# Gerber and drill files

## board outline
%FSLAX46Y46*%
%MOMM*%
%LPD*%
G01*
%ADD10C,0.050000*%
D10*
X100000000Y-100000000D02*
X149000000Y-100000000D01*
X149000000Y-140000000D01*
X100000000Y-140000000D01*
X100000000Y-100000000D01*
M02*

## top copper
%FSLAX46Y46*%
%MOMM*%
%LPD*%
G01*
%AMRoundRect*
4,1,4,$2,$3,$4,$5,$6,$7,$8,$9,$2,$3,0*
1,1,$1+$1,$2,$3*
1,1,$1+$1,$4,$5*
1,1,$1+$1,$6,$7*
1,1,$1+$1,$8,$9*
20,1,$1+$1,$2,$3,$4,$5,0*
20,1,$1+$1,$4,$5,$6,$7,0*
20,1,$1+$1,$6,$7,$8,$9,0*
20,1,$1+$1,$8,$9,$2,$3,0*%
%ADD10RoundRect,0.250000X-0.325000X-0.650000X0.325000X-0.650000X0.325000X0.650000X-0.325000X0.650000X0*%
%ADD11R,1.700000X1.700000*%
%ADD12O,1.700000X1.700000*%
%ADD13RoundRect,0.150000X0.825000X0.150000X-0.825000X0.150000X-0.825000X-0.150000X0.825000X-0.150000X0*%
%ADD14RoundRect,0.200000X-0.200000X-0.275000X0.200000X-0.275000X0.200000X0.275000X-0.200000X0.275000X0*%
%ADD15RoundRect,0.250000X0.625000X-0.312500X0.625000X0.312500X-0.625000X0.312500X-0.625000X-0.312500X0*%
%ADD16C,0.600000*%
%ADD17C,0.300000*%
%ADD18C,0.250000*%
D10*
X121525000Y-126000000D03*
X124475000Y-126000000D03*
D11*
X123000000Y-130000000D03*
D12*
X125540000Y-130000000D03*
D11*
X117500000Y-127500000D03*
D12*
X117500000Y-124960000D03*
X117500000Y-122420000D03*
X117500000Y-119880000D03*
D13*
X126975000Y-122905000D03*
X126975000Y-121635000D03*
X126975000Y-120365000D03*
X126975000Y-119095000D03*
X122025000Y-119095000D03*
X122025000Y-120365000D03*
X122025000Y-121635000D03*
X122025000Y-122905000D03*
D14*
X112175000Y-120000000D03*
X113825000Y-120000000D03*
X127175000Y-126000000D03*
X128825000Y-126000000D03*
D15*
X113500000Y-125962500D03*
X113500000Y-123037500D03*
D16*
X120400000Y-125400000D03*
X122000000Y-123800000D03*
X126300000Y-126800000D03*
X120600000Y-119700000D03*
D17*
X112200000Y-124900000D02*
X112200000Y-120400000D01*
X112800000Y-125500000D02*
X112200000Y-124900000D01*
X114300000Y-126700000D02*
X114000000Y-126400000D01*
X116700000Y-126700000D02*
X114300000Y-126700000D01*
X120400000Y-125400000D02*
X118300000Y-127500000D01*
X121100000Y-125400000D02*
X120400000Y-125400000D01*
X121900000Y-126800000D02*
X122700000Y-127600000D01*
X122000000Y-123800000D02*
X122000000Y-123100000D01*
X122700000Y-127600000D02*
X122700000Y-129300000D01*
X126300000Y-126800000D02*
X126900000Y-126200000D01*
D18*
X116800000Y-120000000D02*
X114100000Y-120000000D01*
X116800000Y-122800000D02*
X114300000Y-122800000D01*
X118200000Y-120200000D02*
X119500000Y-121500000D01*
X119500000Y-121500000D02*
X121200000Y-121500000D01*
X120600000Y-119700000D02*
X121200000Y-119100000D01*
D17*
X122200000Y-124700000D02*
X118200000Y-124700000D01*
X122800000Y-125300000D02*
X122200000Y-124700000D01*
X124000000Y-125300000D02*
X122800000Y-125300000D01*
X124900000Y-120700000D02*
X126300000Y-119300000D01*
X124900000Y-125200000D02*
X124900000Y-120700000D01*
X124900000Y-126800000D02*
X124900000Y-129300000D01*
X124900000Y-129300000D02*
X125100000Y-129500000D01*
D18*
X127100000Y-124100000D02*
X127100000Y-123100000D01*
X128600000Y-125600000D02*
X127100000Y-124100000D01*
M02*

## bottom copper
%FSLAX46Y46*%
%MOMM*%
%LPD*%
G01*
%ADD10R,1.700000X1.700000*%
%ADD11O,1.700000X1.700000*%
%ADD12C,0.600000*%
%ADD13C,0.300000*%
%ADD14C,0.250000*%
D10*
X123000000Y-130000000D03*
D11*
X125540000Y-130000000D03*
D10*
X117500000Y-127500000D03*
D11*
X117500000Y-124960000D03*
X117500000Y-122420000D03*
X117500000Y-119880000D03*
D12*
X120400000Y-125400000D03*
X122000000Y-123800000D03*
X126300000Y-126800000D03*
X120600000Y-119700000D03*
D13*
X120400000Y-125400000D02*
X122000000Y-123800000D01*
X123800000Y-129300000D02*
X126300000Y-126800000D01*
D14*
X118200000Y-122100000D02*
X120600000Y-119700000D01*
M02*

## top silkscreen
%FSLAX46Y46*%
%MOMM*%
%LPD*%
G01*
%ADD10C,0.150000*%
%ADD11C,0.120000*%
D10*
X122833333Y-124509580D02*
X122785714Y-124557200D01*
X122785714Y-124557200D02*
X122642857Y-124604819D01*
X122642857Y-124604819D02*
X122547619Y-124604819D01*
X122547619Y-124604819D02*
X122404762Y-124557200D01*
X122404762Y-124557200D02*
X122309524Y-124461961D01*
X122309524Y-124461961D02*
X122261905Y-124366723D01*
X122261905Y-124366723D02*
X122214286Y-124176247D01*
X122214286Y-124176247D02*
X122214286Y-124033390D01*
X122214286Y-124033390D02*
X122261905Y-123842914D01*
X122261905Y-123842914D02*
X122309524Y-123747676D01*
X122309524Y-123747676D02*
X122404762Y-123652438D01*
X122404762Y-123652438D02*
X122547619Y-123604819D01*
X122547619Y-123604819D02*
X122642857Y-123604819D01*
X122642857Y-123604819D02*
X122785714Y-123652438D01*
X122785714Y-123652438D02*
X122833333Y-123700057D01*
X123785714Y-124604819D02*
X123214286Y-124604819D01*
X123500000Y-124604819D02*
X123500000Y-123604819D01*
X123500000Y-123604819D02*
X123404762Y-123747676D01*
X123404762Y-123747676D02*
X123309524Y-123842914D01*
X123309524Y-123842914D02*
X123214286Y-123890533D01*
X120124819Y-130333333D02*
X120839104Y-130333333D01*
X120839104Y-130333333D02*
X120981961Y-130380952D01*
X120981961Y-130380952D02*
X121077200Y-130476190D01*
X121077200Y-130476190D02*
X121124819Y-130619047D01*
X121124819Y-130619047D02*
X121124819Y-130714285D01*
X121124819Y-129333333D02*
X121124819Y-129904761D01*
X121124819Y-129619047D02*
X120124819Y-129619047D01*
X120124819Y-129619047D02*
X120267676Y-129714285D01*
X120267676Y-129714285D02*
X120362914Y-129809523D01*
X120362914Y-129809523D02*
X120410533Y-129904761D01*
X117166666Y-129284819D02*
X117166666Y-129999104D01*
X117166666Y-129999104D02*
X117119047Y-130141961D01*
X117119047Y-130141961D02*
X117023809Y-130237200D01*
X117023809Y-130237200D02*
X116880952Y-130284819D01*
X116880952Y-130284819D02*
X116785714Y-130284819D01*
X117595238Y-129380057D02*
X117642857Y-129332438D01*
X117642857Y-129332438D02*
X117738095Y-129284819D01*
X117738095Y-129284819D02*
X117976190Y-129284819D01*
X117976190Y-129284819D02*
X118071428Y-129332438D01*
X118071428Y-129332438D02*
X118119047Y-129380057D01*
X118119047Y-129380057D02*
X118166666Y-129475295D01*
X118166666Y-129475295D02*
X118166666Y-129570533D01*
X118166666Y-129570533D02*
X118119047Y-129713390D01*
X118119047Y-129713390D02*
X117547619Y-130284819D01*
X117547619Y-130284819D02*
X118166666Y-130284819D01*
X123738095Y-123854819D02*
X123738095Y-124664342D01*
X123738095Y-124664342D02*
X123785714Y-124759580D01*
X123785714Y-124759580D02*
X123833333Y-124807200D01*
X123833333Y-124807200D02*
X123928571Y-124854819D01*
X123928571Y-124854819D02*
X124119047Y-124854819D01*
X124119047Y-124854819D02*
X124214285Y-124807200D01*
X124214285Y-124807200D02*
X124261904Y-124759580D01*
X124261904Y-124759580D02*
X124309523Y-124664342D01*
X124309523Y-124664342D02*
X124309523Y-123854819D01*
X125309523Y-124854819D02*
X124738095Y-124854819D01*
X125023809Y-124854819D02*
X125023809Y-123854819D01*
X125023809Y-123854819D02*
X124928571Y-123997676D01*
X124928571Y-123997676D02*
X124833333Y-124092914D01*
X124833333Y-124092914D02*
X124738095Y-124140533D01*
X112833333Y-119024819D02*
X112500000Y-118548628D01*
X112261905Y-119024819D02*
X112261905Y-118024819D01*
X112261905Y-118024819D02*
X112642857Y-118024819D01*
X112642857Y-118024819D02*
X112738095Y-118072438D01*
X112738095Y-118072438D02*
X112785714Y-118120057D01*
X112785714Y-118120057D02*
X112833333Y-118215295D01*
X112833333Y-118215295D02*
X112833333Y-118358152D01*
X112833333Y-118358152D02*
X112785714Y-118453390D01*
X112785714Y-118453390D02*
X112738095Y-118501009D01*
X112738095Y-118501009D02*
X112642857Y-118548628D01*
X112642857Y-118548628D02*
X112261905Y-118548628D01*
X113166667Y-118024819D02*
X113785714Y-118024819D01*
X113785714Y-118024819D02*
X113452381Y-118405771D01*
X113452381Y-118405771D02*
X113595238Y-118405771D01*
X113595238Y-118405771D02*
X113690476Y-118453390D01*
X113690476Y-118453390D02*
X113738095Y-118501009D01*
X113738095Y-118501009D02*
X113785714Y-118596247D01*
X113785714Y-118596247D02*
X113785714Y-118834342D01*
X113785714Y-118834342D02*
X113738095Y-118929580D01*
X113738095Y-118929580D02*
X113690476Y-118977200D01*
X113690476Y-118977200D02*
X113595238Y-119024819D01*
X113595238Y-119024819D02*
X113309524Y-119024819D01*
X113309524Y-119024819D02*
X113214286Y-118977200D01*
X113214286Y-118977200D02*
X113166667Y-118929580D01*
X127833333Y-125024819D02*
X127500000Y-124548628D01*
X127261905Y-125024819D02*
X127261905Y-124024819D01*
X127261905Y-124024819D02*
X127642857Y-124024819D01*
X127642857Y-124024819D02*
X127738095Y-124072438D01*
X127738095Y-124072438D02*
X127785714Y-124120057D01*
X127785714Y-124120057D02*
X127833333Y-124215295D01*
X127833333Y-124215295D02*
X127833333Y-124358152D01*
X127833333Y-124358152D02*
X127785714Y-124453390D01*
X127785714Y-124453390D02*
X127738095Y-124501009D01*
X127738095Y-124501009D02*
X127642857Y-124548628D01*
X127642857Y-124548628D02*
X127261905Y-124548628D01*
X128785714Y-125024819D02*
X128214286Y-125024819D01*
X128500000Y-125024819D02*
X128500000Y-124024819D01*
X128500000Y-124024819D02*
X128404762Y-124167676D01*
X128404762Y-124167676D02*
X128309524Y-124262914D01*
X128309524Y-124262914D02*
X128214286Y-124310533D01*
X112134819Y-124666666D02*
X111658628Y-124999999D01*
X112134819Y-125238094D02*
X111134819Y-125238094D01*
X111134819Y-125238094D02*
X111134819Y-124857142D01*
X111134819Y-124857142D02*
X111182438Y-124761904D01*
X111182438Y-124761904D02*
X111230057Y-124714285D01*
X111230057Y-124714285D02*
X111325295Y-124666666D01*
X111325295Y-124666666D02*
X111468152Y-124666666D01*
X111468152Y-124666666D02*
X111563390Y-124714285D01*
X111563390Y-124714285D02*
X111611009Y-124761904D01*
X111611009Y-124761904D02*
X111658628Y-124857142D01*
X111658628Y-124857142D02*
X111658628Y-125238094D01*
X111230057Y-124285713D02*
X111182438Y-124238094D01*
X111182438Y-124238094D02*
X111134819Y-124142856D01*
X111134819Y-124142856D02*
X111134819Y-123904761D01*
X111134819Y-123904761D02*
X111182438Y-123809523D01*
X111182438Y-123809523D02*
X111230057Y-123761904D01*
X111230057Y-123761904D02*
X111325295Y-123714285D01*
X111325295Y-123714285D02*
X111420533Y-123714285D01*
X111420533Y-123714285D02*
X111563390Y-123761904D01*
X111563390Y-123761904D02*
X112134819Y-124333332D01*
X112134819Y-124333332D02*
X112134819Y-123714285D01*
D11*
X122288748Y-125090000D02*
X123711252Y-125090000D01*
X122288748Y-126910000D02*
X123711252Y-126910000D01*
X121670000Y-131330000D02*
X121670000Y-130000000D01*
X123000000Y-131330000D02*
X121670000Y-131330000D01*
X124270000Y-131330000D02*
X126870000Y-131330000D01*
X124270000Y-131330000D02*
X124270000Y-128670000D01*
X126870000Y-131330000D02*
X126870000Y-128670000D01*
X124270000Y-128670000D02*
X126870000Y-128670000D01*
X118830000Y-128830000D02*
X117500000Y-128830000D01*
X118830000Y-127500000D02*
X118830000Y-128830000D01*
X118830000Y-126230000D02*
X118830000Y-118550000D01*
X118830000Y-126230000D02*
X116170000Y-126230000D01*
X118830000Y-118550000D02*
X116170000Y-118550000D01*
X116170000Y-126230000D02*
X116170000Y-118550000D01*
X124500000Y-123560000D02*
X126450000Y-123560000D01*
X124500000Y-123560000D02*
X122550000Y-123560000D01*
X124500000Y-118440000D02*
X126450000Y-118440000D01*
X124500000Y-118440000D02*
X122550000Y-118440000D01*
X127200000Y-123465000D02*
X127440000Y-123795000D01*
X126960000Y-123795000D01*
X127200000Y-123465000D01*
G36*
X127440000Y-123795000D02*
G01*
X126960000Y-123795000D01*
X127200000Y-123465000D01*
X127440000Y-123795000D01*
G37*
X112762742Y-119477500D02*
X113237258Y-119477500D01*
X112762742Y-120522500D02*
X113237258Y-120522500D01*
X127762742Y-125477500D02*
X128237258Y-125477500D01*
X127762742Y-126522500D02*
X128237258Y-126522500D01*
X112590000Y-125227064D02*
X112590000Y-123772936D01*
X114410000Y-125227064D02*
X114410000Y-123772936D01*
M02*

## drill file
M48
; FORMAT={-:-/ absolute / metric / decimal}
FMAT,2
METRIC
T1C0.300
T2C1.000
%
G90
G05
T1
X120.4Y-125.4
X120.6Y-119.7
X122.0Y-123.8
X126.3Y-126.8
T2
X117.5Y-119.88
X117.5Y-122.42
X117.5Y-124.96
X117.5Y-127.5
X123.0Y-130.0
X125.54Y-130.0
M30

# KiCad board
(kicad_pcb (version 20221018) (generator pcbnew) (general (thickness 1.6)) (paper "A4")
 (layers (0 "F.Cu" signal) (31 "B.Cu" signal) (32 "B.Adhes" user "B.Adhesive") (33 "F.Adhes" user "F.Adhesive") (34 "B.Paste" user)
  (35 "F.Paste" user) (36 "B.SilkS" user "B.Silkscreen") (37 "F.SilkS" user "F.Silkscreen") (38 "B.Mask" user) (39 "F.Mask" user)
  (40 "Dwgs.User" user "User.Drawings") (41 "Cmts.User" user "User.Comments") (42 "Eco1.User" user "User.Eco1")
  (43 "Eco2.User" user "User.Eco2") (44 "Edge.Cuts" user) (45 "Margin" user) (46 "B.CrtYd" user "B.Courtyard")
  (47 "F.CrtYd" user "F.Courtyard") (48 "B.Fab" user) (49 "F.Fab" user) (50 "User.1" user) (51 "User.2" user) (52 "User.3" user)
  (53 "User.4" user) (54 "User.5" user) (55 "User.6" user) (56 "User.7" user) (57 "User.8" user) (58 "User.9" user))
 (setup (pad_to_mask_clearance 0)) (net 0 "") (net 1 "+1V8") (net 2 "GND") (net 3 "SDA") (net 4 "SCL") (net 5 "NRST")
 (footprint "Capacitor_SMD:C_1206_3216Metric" (layer "F.Cu") (at 123 126)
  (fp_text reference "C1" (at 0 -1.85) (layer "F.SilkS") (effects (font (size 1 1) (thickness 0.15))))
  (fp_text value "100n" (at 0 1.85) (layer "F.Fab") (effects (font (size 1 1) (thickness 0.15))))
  (fp_line (start -0.711252 -0.91) (end 0.711252 -0.91) (stroke (width 0.12) (type solid)) (layer "F.SilkS"))
  (fp_line (start -0.711252 0.91) (end 0.711252 0.91) (stroke (width 0.12) (type solid)) (layer "F.SilkS"))
  (pad "1" smd roundrect (at -1.475 0) (size 1.15 1.8) (layers "F.Cu" "F.Paste" "F.Mask") (roundrect_rratio 0.217391) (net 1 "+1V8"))
  (pad "2" smd roundrect (at 1.475 0) (size 1.15 1.8) (layers "F.Cu" "F.Paste" "F.Mask") (roundrect_rratio 0.217391) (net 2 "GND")))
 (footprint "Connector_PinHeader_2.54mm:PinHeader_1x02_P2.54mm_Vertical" (layer "F.Cu") (at 123 130 90)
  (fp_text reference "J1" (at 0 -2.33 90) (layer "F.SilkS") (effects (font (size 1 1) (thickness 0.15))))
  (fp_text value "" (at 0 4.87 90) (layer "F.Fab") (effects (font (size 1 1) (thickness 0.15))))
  (fp_line (start -1.33 -1.33) (end 0 -1.33) (stroke (width 0.12) (type solid)) (layer "F.SilkS"))
  (fp_line (start -1.33 0) (end -1.33 -1.33) (stroke (width 0.12) (type solid)) (layer "F.SilkS"))
  (fp_line (start -1.33 1.27) (end -1.33 3.87) (stroke (width 0.12) (type solid)) (layer "F.SilkS"))
  (fp_line (start -1.33 1.27) (end 1.33 1.27) (stroke (width 0.12) (type solid)) (layer "F.SilkS"))
  (fp_line (start -1.33 3.87) (end 1.33 3.87) (stroke (width 0.12) (type solid)) (layer "F.SilkS"))
  (fp_line (start 1.33 1.27) (end 1.33 3.87) (stroke (width 0.12) (type solid)) (layer "F.SilkS"))
  (pad "1" thru_hole rect (at 0 0 90) (size 1.7 1.7) (drill 1) (layers "*.Cu" "*.Mask") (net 1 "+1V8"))
  (pad "2" thru_hole oval (at 0 2.54 90) (size 1.7 1.7) (drill 1) (layers "*.Cu" "*.Mask") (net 2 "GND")))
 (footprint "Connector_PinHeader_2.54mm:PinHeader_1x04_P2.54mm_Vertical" (layer "F.Cu") (at 117.5 127.5 180)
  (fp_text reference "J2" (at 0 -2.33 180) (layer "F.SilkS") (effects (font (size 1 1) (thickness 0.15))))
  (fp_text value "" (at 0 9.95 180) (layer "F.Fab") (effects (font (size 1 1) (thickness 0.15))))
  (fp_line (start -1.33 -1.33) (end 0 -1.33) (stroke (width 0.12) (type solid)) (layer "F.SilkS"))
  (fp_line (start -1.33 0) (end -1.33 -1.33) (stroke (width 0.12) (type solid)) (layer "F.SilkS"))
  (fp_line (start -1.33 1.27) (end -1.33 8.95) (stroke (width 0.12) (type solid)) (layer "F.SilkS"))
  (fp_line (start -1.33 1.27) (end 1.33 1.27) (stroke (width 0.12) (type solid)) (layer "F.SilkS"))
  (fp_line (start -1.33 8.95) (end 1.33 8.95) (stroke (width 0.12) (type solid)) (layer "F.SilkS"))
  (fp_line (start 1.33 1.27) (end 1.33 8.95) (stroke (width 0.12) (type solid)) (layer "F.SilkS"))
  (pad "1" thru_hole rect (at 0 0 180) (size 1.7 1.7) (drill 1) (layers "*.Cu" "*.Mask") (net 1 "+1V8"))
  (pad "2" thru_hole oval (at 0 2.54 180) (size 1.7 1.7) (drill 1) (layers "*.Cu" "*.Mask") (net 2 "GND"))
  (pad "3" thru_hole oval (at 0 5.08 180) (size 1.7 1.7) (drill 1) (layers "*.Cu" "*.Mask") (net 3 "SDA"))
  (pad "4" thru_hole oval (at 0 7.62 180) (size 1.7 1.7) (drill 1) (layers "*.Cu" "*.Mask") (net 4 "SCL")))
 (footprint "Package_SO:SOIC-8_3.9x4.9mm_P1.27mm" (layer "F.Cu") (at 124.5 121 180)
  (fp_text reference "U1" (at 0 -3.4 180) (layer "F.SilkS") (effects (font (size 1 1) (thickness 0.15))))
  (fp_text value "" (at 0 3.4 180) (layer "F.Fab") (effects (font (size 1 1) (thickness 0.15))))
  (fp_line (start 0 -2.56) (end -1.95 -2.56) (stroke (width 0.12) (type solid)) (layer "F.SilkS"))
  (fp_line (start 0 -2.56) (end 1.95 -2.56) (stroke (width 0.12) (type solid)) (layer "F.SilkS"))
  (fp_line (start 0 2.56) (end -1.95 2.56) (stroke (width 0.12) (type solid)) (layer "F.SilkS"))
  (fp_line (start 0 2.56) (end 1.95 2.56) (stroke (width 0.12) (type solid)) (layer "F.SilkS"))
  (fp_poly
   (pts (xy -2.7 -2.465) (xy -2.94 -2.795) (xy -2.46 -2.795) (xy -2.7 -2.465)) (stroke (width 0.12) (type solid)) (fill solid)
   (layer "F.SilkS"))
  (pad "1" smd roundrect (at -2.475 -1.905 180) (size 1.95 0.6) (layers "F.Cu" "F.Paste" "F.Mask") (roundrect_rratio 0.25) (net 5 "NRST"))
  (pad "2" smd roundrect (at -2.475 -0.635 180) (size 1.95 0.6) (layers "F.Cu" "F.Paste" "F.Mask") (roundrect_rratio 0.25))
  (pad "3" smd roundrect (at -2.475 0.635 180) (size 1.95 0.6) (layers "F.Cu" "F.Paste" "F.Mask") (roundrect_rratio 0.25))
  (pad "4" smd roundrect (at -2.475 1.905 180) (size 1.95 0.6) (layers "F.Cu" "F.Paste" "F.Mask") (roundrect_rratio 0.25) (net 2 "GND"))
  (pad "5" smd roundrect (at 2.475 1.905 180) (size 1.95 0.6) (layers "F.Cu" "F.Paste" "F.Mask") (roundrect_rratio 0.25) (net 3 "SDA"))
  (pad "6" smd roundrect (at 2.475 0.635 180) (size 1.95 0.6) (layers "F.Cu" "F.Paste" "F.Mask") (roundrect_rratio 0.25))
  (pad "7" smd roundrect (at 2.475 -0.635 180) (size 1.95 0.6) (layers "F.Cu" "F.Paste" "F.Mask") (roundrect_rratio 0.25) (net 4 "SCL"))
  (pad "8" smd roundrect (at 2.475 -1.905 180) (size 1.95 0.6) (layers "F.Cu" "F.Paste" "F.Mask") (roundrect_rratio 0.25) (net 1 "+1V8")))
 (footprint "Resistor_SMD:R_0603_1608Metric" (layer "F.Cu") (at 113 120)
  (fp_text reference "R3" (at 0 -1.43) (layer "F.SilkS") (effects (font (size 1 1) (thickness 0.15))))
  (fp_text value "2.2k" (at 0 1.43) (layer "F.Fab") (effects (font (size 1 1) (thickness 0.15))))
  (fp_line (start -0.237258 -0.5225) (end 0.237258 -0.5225) (stroke (width 0.12) (type solid)) (layer "F.SilkS"))
  (fp_line (start -0.237258 0.5225) (end 0.237258 0.5225) (stroke (width 0.12) (type solid)) (layer "F.SilkS"))
  (pad "1" smd roundrect (at -0.825 0) (size 0.8 0.95) (layers "F.Cu" "F.Paste" "F.Mask") (roundrect_rratio 0.25) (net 1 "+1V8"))
  (pad "2" smd roundrect (at 0.825 0) (size 0.8 0.95) (layers "F.Cu" "F.Paste" "F.Mask") (roundrect_rratio 0.25) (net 4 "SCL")))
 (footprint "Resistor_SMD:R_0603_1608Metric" (layer "F.Cu") (at 128 126)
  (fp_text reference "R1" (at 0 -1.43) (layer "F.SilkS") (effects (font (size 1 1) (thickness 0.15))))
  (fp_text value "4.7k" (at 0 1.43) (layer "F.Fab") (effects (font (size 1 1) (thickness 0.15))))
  (fp_line (start -0.237258 -0.5225) (end 0.237258 -0.5225) (stroke (width 0.12) (type solid)) (layer "F.SilkS"))
  (fp_line (start -0.237258 0.5225) (end 0.237258 0.5225) (stroke (width 0.12) (type solid)) (layer "F.SilkS"))
  (pad "1" smd roundrect (at -0.825 0) (size 0.8 0.95) (layers "F.Cu" "F.Paste" "F.Mask") (roundrect_rratio 0.25) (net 1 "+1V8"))
  (pad "2" smd roundrect (at 0.825 0) (size 0.8 0.95) (layers "F.Cu" "F.Paste" "F.Mask") (roundrect_rratio 0.25) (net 5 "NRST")))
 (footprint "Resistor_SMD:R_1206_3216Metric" (layer "F.Cu") (at 113.5 124.5 90)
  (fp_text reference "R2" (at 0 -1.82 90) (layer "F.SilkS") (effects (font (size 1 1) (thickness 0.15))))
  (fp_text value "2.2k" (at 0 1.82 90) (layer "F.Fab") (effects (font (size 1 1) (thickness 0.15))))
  (fp_line (start -0.727064 -0.91) (end 0.727064 -0.91) (stroke (width 0.12) (type solid)) (layer "F.SilkS"))
  (fp_line (start -0.727064 0.91) (end 0.727064 0.91) (stroke (width 0.12) (type solid)) (layer "F.SilkS"))
  (pad "1" smd roundrect (at -1.4625 0 90) (size 1.125 1.75) (layers "F.Cu" "F.Paste" "F.Mask") (roundrect_rratio 0.222222) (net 1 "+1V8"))
  (pad "2" smd roundrect (at 1.4625 0 90) (size 1.125 1.75) (layers "F.Cu" "F.Paste" "F.Mask") (roundrect_rratio 0.222222) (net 3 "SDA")))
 (gr_rect (start 100 100) (end 149 140) (stroke (width 0.05) (type default)) (fill none) (layer "Edge.Cuts"))
 (segment (start 112.2 124.9) (end 112.2 120.4) (width 0.3) (layer "F.Cu") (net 1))
 (segment (start 112.8 125.5) (end 112.2 124.9) (width 0.3) (layer "F.Cu") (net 1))
 (segment (start 114.3 126.7) (end 114 126.4) (width 0.3) (layer "F.Cu") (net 1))
 (segment (start 116.7 126.7) (end 114.3 126.7) (width 0.3) (layer "F.Cu") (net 1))
 (segment (start 120.4 125.4) (end 118.3 127.5) (width 0.3) (layer "F.Cu") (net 1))
 (segment (start 121.1 125.4) (end 120.4 125.4) (width 0.3) (layer "F.Cu") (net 1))
 (segment (start 121.9 126.8) (end 122.7 127.6) (width 0.3) (layer "F.Cu") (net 1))
 (segment (start 122 123.8) (end 122 123.1) (width 0.3) (layer "F.Cu") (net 1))
 (segment (start 122.7 127.6) (end 122.7 129.3) (width 0.3) (layer "F.Cu") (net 1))
 (segment (start 126.3 126.8) (end 126.9 126.2) (width 0.3) (layer "F.Cu") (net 1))
 (via (at 120.4 125.4) (size 0.6) (drill 0.3) (layers "F.Cu" "B.Cu") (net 1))
 (via (at 122 123.8) (size 0.6) (drill 0.3) (layers "F.Cu" "B.Cu") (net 1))
 (via (at 126.3 126.8) (size 0.6) (drill 0.3) (layers "F.Cu" "B.Cu") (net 1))
 (segment (start 116.8 120) (end 114.1 120) (width 0.25) (layer "F.Cu") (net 4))
 (segment (start 116.8 122.8) (end 114.3 122.8) (width 0.25) (layer "F.Cu") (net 3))
 (segment (start 118.2 120.2) (end 119.5 121.5) (width 0.25) (layer "F.Cu") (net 4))
 (segment (start 119.5 121.5) (end 121.2 121.5) (width 0.25) (layer "F.Cu") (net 4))
 (segment (start 120.4 125.4) (end 122 123.8) (width 0.3) (layer "B.Cu") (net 1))
 (segment (start 120.6 119.7) (end 121.2 119.1) (width 0.25) (layer "F.Cu") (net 3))
 (segment (start 122.2 124.7) (end 118.2 124.7) (width 0.3) (layer "F.Cu") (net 2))
 (segment (start 122.8 125.3) (end 122.2 124.7) (width 0.3) (layer "F.Cu") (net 2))
 (segment (start 123.8 129.3) (end 126.3 126.8) (width 0.3) (layer "B.Cu") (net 1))
 (segment (start 124 125.3) (end 122.8 125.3) (width 0.3) (layer "F.Cu") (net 2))
 (segment (start 124.9 120.7) (end 126.3 119.3) (width 0.3) (layer "F.Cu") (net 2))
 (segment (start 124.9 125.2) (end 124.9 120.7) (width 0.3) (layer "F.Cu") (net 2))
 (segment (start 124.9 126.8) (end 124.9 129.3) (width 0.3) (layer "F.Cu") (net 2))
 (segment (start 124.9 129.3) (end 125.1 129.5) (width 0.3) (layer "F.Cu") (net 2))
 (segment (start 127.1 124.1) (end 127.1 123.1) (width 0.25) (layer "F.Cu") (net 5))
 (segment (start 128.6 125.6) (end 127.1 124.1) (width 0.25) (layer "F.Cu") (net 5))
 (via (at 120.6 119.7) (size 0.6) (drill 0.3) (layers "F.Cu" "B.Cu") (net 3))
 (segment (start 118.2 122.1) (end 120.6 119.7) (width 0.25) (layer "B.Cu") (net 3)))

